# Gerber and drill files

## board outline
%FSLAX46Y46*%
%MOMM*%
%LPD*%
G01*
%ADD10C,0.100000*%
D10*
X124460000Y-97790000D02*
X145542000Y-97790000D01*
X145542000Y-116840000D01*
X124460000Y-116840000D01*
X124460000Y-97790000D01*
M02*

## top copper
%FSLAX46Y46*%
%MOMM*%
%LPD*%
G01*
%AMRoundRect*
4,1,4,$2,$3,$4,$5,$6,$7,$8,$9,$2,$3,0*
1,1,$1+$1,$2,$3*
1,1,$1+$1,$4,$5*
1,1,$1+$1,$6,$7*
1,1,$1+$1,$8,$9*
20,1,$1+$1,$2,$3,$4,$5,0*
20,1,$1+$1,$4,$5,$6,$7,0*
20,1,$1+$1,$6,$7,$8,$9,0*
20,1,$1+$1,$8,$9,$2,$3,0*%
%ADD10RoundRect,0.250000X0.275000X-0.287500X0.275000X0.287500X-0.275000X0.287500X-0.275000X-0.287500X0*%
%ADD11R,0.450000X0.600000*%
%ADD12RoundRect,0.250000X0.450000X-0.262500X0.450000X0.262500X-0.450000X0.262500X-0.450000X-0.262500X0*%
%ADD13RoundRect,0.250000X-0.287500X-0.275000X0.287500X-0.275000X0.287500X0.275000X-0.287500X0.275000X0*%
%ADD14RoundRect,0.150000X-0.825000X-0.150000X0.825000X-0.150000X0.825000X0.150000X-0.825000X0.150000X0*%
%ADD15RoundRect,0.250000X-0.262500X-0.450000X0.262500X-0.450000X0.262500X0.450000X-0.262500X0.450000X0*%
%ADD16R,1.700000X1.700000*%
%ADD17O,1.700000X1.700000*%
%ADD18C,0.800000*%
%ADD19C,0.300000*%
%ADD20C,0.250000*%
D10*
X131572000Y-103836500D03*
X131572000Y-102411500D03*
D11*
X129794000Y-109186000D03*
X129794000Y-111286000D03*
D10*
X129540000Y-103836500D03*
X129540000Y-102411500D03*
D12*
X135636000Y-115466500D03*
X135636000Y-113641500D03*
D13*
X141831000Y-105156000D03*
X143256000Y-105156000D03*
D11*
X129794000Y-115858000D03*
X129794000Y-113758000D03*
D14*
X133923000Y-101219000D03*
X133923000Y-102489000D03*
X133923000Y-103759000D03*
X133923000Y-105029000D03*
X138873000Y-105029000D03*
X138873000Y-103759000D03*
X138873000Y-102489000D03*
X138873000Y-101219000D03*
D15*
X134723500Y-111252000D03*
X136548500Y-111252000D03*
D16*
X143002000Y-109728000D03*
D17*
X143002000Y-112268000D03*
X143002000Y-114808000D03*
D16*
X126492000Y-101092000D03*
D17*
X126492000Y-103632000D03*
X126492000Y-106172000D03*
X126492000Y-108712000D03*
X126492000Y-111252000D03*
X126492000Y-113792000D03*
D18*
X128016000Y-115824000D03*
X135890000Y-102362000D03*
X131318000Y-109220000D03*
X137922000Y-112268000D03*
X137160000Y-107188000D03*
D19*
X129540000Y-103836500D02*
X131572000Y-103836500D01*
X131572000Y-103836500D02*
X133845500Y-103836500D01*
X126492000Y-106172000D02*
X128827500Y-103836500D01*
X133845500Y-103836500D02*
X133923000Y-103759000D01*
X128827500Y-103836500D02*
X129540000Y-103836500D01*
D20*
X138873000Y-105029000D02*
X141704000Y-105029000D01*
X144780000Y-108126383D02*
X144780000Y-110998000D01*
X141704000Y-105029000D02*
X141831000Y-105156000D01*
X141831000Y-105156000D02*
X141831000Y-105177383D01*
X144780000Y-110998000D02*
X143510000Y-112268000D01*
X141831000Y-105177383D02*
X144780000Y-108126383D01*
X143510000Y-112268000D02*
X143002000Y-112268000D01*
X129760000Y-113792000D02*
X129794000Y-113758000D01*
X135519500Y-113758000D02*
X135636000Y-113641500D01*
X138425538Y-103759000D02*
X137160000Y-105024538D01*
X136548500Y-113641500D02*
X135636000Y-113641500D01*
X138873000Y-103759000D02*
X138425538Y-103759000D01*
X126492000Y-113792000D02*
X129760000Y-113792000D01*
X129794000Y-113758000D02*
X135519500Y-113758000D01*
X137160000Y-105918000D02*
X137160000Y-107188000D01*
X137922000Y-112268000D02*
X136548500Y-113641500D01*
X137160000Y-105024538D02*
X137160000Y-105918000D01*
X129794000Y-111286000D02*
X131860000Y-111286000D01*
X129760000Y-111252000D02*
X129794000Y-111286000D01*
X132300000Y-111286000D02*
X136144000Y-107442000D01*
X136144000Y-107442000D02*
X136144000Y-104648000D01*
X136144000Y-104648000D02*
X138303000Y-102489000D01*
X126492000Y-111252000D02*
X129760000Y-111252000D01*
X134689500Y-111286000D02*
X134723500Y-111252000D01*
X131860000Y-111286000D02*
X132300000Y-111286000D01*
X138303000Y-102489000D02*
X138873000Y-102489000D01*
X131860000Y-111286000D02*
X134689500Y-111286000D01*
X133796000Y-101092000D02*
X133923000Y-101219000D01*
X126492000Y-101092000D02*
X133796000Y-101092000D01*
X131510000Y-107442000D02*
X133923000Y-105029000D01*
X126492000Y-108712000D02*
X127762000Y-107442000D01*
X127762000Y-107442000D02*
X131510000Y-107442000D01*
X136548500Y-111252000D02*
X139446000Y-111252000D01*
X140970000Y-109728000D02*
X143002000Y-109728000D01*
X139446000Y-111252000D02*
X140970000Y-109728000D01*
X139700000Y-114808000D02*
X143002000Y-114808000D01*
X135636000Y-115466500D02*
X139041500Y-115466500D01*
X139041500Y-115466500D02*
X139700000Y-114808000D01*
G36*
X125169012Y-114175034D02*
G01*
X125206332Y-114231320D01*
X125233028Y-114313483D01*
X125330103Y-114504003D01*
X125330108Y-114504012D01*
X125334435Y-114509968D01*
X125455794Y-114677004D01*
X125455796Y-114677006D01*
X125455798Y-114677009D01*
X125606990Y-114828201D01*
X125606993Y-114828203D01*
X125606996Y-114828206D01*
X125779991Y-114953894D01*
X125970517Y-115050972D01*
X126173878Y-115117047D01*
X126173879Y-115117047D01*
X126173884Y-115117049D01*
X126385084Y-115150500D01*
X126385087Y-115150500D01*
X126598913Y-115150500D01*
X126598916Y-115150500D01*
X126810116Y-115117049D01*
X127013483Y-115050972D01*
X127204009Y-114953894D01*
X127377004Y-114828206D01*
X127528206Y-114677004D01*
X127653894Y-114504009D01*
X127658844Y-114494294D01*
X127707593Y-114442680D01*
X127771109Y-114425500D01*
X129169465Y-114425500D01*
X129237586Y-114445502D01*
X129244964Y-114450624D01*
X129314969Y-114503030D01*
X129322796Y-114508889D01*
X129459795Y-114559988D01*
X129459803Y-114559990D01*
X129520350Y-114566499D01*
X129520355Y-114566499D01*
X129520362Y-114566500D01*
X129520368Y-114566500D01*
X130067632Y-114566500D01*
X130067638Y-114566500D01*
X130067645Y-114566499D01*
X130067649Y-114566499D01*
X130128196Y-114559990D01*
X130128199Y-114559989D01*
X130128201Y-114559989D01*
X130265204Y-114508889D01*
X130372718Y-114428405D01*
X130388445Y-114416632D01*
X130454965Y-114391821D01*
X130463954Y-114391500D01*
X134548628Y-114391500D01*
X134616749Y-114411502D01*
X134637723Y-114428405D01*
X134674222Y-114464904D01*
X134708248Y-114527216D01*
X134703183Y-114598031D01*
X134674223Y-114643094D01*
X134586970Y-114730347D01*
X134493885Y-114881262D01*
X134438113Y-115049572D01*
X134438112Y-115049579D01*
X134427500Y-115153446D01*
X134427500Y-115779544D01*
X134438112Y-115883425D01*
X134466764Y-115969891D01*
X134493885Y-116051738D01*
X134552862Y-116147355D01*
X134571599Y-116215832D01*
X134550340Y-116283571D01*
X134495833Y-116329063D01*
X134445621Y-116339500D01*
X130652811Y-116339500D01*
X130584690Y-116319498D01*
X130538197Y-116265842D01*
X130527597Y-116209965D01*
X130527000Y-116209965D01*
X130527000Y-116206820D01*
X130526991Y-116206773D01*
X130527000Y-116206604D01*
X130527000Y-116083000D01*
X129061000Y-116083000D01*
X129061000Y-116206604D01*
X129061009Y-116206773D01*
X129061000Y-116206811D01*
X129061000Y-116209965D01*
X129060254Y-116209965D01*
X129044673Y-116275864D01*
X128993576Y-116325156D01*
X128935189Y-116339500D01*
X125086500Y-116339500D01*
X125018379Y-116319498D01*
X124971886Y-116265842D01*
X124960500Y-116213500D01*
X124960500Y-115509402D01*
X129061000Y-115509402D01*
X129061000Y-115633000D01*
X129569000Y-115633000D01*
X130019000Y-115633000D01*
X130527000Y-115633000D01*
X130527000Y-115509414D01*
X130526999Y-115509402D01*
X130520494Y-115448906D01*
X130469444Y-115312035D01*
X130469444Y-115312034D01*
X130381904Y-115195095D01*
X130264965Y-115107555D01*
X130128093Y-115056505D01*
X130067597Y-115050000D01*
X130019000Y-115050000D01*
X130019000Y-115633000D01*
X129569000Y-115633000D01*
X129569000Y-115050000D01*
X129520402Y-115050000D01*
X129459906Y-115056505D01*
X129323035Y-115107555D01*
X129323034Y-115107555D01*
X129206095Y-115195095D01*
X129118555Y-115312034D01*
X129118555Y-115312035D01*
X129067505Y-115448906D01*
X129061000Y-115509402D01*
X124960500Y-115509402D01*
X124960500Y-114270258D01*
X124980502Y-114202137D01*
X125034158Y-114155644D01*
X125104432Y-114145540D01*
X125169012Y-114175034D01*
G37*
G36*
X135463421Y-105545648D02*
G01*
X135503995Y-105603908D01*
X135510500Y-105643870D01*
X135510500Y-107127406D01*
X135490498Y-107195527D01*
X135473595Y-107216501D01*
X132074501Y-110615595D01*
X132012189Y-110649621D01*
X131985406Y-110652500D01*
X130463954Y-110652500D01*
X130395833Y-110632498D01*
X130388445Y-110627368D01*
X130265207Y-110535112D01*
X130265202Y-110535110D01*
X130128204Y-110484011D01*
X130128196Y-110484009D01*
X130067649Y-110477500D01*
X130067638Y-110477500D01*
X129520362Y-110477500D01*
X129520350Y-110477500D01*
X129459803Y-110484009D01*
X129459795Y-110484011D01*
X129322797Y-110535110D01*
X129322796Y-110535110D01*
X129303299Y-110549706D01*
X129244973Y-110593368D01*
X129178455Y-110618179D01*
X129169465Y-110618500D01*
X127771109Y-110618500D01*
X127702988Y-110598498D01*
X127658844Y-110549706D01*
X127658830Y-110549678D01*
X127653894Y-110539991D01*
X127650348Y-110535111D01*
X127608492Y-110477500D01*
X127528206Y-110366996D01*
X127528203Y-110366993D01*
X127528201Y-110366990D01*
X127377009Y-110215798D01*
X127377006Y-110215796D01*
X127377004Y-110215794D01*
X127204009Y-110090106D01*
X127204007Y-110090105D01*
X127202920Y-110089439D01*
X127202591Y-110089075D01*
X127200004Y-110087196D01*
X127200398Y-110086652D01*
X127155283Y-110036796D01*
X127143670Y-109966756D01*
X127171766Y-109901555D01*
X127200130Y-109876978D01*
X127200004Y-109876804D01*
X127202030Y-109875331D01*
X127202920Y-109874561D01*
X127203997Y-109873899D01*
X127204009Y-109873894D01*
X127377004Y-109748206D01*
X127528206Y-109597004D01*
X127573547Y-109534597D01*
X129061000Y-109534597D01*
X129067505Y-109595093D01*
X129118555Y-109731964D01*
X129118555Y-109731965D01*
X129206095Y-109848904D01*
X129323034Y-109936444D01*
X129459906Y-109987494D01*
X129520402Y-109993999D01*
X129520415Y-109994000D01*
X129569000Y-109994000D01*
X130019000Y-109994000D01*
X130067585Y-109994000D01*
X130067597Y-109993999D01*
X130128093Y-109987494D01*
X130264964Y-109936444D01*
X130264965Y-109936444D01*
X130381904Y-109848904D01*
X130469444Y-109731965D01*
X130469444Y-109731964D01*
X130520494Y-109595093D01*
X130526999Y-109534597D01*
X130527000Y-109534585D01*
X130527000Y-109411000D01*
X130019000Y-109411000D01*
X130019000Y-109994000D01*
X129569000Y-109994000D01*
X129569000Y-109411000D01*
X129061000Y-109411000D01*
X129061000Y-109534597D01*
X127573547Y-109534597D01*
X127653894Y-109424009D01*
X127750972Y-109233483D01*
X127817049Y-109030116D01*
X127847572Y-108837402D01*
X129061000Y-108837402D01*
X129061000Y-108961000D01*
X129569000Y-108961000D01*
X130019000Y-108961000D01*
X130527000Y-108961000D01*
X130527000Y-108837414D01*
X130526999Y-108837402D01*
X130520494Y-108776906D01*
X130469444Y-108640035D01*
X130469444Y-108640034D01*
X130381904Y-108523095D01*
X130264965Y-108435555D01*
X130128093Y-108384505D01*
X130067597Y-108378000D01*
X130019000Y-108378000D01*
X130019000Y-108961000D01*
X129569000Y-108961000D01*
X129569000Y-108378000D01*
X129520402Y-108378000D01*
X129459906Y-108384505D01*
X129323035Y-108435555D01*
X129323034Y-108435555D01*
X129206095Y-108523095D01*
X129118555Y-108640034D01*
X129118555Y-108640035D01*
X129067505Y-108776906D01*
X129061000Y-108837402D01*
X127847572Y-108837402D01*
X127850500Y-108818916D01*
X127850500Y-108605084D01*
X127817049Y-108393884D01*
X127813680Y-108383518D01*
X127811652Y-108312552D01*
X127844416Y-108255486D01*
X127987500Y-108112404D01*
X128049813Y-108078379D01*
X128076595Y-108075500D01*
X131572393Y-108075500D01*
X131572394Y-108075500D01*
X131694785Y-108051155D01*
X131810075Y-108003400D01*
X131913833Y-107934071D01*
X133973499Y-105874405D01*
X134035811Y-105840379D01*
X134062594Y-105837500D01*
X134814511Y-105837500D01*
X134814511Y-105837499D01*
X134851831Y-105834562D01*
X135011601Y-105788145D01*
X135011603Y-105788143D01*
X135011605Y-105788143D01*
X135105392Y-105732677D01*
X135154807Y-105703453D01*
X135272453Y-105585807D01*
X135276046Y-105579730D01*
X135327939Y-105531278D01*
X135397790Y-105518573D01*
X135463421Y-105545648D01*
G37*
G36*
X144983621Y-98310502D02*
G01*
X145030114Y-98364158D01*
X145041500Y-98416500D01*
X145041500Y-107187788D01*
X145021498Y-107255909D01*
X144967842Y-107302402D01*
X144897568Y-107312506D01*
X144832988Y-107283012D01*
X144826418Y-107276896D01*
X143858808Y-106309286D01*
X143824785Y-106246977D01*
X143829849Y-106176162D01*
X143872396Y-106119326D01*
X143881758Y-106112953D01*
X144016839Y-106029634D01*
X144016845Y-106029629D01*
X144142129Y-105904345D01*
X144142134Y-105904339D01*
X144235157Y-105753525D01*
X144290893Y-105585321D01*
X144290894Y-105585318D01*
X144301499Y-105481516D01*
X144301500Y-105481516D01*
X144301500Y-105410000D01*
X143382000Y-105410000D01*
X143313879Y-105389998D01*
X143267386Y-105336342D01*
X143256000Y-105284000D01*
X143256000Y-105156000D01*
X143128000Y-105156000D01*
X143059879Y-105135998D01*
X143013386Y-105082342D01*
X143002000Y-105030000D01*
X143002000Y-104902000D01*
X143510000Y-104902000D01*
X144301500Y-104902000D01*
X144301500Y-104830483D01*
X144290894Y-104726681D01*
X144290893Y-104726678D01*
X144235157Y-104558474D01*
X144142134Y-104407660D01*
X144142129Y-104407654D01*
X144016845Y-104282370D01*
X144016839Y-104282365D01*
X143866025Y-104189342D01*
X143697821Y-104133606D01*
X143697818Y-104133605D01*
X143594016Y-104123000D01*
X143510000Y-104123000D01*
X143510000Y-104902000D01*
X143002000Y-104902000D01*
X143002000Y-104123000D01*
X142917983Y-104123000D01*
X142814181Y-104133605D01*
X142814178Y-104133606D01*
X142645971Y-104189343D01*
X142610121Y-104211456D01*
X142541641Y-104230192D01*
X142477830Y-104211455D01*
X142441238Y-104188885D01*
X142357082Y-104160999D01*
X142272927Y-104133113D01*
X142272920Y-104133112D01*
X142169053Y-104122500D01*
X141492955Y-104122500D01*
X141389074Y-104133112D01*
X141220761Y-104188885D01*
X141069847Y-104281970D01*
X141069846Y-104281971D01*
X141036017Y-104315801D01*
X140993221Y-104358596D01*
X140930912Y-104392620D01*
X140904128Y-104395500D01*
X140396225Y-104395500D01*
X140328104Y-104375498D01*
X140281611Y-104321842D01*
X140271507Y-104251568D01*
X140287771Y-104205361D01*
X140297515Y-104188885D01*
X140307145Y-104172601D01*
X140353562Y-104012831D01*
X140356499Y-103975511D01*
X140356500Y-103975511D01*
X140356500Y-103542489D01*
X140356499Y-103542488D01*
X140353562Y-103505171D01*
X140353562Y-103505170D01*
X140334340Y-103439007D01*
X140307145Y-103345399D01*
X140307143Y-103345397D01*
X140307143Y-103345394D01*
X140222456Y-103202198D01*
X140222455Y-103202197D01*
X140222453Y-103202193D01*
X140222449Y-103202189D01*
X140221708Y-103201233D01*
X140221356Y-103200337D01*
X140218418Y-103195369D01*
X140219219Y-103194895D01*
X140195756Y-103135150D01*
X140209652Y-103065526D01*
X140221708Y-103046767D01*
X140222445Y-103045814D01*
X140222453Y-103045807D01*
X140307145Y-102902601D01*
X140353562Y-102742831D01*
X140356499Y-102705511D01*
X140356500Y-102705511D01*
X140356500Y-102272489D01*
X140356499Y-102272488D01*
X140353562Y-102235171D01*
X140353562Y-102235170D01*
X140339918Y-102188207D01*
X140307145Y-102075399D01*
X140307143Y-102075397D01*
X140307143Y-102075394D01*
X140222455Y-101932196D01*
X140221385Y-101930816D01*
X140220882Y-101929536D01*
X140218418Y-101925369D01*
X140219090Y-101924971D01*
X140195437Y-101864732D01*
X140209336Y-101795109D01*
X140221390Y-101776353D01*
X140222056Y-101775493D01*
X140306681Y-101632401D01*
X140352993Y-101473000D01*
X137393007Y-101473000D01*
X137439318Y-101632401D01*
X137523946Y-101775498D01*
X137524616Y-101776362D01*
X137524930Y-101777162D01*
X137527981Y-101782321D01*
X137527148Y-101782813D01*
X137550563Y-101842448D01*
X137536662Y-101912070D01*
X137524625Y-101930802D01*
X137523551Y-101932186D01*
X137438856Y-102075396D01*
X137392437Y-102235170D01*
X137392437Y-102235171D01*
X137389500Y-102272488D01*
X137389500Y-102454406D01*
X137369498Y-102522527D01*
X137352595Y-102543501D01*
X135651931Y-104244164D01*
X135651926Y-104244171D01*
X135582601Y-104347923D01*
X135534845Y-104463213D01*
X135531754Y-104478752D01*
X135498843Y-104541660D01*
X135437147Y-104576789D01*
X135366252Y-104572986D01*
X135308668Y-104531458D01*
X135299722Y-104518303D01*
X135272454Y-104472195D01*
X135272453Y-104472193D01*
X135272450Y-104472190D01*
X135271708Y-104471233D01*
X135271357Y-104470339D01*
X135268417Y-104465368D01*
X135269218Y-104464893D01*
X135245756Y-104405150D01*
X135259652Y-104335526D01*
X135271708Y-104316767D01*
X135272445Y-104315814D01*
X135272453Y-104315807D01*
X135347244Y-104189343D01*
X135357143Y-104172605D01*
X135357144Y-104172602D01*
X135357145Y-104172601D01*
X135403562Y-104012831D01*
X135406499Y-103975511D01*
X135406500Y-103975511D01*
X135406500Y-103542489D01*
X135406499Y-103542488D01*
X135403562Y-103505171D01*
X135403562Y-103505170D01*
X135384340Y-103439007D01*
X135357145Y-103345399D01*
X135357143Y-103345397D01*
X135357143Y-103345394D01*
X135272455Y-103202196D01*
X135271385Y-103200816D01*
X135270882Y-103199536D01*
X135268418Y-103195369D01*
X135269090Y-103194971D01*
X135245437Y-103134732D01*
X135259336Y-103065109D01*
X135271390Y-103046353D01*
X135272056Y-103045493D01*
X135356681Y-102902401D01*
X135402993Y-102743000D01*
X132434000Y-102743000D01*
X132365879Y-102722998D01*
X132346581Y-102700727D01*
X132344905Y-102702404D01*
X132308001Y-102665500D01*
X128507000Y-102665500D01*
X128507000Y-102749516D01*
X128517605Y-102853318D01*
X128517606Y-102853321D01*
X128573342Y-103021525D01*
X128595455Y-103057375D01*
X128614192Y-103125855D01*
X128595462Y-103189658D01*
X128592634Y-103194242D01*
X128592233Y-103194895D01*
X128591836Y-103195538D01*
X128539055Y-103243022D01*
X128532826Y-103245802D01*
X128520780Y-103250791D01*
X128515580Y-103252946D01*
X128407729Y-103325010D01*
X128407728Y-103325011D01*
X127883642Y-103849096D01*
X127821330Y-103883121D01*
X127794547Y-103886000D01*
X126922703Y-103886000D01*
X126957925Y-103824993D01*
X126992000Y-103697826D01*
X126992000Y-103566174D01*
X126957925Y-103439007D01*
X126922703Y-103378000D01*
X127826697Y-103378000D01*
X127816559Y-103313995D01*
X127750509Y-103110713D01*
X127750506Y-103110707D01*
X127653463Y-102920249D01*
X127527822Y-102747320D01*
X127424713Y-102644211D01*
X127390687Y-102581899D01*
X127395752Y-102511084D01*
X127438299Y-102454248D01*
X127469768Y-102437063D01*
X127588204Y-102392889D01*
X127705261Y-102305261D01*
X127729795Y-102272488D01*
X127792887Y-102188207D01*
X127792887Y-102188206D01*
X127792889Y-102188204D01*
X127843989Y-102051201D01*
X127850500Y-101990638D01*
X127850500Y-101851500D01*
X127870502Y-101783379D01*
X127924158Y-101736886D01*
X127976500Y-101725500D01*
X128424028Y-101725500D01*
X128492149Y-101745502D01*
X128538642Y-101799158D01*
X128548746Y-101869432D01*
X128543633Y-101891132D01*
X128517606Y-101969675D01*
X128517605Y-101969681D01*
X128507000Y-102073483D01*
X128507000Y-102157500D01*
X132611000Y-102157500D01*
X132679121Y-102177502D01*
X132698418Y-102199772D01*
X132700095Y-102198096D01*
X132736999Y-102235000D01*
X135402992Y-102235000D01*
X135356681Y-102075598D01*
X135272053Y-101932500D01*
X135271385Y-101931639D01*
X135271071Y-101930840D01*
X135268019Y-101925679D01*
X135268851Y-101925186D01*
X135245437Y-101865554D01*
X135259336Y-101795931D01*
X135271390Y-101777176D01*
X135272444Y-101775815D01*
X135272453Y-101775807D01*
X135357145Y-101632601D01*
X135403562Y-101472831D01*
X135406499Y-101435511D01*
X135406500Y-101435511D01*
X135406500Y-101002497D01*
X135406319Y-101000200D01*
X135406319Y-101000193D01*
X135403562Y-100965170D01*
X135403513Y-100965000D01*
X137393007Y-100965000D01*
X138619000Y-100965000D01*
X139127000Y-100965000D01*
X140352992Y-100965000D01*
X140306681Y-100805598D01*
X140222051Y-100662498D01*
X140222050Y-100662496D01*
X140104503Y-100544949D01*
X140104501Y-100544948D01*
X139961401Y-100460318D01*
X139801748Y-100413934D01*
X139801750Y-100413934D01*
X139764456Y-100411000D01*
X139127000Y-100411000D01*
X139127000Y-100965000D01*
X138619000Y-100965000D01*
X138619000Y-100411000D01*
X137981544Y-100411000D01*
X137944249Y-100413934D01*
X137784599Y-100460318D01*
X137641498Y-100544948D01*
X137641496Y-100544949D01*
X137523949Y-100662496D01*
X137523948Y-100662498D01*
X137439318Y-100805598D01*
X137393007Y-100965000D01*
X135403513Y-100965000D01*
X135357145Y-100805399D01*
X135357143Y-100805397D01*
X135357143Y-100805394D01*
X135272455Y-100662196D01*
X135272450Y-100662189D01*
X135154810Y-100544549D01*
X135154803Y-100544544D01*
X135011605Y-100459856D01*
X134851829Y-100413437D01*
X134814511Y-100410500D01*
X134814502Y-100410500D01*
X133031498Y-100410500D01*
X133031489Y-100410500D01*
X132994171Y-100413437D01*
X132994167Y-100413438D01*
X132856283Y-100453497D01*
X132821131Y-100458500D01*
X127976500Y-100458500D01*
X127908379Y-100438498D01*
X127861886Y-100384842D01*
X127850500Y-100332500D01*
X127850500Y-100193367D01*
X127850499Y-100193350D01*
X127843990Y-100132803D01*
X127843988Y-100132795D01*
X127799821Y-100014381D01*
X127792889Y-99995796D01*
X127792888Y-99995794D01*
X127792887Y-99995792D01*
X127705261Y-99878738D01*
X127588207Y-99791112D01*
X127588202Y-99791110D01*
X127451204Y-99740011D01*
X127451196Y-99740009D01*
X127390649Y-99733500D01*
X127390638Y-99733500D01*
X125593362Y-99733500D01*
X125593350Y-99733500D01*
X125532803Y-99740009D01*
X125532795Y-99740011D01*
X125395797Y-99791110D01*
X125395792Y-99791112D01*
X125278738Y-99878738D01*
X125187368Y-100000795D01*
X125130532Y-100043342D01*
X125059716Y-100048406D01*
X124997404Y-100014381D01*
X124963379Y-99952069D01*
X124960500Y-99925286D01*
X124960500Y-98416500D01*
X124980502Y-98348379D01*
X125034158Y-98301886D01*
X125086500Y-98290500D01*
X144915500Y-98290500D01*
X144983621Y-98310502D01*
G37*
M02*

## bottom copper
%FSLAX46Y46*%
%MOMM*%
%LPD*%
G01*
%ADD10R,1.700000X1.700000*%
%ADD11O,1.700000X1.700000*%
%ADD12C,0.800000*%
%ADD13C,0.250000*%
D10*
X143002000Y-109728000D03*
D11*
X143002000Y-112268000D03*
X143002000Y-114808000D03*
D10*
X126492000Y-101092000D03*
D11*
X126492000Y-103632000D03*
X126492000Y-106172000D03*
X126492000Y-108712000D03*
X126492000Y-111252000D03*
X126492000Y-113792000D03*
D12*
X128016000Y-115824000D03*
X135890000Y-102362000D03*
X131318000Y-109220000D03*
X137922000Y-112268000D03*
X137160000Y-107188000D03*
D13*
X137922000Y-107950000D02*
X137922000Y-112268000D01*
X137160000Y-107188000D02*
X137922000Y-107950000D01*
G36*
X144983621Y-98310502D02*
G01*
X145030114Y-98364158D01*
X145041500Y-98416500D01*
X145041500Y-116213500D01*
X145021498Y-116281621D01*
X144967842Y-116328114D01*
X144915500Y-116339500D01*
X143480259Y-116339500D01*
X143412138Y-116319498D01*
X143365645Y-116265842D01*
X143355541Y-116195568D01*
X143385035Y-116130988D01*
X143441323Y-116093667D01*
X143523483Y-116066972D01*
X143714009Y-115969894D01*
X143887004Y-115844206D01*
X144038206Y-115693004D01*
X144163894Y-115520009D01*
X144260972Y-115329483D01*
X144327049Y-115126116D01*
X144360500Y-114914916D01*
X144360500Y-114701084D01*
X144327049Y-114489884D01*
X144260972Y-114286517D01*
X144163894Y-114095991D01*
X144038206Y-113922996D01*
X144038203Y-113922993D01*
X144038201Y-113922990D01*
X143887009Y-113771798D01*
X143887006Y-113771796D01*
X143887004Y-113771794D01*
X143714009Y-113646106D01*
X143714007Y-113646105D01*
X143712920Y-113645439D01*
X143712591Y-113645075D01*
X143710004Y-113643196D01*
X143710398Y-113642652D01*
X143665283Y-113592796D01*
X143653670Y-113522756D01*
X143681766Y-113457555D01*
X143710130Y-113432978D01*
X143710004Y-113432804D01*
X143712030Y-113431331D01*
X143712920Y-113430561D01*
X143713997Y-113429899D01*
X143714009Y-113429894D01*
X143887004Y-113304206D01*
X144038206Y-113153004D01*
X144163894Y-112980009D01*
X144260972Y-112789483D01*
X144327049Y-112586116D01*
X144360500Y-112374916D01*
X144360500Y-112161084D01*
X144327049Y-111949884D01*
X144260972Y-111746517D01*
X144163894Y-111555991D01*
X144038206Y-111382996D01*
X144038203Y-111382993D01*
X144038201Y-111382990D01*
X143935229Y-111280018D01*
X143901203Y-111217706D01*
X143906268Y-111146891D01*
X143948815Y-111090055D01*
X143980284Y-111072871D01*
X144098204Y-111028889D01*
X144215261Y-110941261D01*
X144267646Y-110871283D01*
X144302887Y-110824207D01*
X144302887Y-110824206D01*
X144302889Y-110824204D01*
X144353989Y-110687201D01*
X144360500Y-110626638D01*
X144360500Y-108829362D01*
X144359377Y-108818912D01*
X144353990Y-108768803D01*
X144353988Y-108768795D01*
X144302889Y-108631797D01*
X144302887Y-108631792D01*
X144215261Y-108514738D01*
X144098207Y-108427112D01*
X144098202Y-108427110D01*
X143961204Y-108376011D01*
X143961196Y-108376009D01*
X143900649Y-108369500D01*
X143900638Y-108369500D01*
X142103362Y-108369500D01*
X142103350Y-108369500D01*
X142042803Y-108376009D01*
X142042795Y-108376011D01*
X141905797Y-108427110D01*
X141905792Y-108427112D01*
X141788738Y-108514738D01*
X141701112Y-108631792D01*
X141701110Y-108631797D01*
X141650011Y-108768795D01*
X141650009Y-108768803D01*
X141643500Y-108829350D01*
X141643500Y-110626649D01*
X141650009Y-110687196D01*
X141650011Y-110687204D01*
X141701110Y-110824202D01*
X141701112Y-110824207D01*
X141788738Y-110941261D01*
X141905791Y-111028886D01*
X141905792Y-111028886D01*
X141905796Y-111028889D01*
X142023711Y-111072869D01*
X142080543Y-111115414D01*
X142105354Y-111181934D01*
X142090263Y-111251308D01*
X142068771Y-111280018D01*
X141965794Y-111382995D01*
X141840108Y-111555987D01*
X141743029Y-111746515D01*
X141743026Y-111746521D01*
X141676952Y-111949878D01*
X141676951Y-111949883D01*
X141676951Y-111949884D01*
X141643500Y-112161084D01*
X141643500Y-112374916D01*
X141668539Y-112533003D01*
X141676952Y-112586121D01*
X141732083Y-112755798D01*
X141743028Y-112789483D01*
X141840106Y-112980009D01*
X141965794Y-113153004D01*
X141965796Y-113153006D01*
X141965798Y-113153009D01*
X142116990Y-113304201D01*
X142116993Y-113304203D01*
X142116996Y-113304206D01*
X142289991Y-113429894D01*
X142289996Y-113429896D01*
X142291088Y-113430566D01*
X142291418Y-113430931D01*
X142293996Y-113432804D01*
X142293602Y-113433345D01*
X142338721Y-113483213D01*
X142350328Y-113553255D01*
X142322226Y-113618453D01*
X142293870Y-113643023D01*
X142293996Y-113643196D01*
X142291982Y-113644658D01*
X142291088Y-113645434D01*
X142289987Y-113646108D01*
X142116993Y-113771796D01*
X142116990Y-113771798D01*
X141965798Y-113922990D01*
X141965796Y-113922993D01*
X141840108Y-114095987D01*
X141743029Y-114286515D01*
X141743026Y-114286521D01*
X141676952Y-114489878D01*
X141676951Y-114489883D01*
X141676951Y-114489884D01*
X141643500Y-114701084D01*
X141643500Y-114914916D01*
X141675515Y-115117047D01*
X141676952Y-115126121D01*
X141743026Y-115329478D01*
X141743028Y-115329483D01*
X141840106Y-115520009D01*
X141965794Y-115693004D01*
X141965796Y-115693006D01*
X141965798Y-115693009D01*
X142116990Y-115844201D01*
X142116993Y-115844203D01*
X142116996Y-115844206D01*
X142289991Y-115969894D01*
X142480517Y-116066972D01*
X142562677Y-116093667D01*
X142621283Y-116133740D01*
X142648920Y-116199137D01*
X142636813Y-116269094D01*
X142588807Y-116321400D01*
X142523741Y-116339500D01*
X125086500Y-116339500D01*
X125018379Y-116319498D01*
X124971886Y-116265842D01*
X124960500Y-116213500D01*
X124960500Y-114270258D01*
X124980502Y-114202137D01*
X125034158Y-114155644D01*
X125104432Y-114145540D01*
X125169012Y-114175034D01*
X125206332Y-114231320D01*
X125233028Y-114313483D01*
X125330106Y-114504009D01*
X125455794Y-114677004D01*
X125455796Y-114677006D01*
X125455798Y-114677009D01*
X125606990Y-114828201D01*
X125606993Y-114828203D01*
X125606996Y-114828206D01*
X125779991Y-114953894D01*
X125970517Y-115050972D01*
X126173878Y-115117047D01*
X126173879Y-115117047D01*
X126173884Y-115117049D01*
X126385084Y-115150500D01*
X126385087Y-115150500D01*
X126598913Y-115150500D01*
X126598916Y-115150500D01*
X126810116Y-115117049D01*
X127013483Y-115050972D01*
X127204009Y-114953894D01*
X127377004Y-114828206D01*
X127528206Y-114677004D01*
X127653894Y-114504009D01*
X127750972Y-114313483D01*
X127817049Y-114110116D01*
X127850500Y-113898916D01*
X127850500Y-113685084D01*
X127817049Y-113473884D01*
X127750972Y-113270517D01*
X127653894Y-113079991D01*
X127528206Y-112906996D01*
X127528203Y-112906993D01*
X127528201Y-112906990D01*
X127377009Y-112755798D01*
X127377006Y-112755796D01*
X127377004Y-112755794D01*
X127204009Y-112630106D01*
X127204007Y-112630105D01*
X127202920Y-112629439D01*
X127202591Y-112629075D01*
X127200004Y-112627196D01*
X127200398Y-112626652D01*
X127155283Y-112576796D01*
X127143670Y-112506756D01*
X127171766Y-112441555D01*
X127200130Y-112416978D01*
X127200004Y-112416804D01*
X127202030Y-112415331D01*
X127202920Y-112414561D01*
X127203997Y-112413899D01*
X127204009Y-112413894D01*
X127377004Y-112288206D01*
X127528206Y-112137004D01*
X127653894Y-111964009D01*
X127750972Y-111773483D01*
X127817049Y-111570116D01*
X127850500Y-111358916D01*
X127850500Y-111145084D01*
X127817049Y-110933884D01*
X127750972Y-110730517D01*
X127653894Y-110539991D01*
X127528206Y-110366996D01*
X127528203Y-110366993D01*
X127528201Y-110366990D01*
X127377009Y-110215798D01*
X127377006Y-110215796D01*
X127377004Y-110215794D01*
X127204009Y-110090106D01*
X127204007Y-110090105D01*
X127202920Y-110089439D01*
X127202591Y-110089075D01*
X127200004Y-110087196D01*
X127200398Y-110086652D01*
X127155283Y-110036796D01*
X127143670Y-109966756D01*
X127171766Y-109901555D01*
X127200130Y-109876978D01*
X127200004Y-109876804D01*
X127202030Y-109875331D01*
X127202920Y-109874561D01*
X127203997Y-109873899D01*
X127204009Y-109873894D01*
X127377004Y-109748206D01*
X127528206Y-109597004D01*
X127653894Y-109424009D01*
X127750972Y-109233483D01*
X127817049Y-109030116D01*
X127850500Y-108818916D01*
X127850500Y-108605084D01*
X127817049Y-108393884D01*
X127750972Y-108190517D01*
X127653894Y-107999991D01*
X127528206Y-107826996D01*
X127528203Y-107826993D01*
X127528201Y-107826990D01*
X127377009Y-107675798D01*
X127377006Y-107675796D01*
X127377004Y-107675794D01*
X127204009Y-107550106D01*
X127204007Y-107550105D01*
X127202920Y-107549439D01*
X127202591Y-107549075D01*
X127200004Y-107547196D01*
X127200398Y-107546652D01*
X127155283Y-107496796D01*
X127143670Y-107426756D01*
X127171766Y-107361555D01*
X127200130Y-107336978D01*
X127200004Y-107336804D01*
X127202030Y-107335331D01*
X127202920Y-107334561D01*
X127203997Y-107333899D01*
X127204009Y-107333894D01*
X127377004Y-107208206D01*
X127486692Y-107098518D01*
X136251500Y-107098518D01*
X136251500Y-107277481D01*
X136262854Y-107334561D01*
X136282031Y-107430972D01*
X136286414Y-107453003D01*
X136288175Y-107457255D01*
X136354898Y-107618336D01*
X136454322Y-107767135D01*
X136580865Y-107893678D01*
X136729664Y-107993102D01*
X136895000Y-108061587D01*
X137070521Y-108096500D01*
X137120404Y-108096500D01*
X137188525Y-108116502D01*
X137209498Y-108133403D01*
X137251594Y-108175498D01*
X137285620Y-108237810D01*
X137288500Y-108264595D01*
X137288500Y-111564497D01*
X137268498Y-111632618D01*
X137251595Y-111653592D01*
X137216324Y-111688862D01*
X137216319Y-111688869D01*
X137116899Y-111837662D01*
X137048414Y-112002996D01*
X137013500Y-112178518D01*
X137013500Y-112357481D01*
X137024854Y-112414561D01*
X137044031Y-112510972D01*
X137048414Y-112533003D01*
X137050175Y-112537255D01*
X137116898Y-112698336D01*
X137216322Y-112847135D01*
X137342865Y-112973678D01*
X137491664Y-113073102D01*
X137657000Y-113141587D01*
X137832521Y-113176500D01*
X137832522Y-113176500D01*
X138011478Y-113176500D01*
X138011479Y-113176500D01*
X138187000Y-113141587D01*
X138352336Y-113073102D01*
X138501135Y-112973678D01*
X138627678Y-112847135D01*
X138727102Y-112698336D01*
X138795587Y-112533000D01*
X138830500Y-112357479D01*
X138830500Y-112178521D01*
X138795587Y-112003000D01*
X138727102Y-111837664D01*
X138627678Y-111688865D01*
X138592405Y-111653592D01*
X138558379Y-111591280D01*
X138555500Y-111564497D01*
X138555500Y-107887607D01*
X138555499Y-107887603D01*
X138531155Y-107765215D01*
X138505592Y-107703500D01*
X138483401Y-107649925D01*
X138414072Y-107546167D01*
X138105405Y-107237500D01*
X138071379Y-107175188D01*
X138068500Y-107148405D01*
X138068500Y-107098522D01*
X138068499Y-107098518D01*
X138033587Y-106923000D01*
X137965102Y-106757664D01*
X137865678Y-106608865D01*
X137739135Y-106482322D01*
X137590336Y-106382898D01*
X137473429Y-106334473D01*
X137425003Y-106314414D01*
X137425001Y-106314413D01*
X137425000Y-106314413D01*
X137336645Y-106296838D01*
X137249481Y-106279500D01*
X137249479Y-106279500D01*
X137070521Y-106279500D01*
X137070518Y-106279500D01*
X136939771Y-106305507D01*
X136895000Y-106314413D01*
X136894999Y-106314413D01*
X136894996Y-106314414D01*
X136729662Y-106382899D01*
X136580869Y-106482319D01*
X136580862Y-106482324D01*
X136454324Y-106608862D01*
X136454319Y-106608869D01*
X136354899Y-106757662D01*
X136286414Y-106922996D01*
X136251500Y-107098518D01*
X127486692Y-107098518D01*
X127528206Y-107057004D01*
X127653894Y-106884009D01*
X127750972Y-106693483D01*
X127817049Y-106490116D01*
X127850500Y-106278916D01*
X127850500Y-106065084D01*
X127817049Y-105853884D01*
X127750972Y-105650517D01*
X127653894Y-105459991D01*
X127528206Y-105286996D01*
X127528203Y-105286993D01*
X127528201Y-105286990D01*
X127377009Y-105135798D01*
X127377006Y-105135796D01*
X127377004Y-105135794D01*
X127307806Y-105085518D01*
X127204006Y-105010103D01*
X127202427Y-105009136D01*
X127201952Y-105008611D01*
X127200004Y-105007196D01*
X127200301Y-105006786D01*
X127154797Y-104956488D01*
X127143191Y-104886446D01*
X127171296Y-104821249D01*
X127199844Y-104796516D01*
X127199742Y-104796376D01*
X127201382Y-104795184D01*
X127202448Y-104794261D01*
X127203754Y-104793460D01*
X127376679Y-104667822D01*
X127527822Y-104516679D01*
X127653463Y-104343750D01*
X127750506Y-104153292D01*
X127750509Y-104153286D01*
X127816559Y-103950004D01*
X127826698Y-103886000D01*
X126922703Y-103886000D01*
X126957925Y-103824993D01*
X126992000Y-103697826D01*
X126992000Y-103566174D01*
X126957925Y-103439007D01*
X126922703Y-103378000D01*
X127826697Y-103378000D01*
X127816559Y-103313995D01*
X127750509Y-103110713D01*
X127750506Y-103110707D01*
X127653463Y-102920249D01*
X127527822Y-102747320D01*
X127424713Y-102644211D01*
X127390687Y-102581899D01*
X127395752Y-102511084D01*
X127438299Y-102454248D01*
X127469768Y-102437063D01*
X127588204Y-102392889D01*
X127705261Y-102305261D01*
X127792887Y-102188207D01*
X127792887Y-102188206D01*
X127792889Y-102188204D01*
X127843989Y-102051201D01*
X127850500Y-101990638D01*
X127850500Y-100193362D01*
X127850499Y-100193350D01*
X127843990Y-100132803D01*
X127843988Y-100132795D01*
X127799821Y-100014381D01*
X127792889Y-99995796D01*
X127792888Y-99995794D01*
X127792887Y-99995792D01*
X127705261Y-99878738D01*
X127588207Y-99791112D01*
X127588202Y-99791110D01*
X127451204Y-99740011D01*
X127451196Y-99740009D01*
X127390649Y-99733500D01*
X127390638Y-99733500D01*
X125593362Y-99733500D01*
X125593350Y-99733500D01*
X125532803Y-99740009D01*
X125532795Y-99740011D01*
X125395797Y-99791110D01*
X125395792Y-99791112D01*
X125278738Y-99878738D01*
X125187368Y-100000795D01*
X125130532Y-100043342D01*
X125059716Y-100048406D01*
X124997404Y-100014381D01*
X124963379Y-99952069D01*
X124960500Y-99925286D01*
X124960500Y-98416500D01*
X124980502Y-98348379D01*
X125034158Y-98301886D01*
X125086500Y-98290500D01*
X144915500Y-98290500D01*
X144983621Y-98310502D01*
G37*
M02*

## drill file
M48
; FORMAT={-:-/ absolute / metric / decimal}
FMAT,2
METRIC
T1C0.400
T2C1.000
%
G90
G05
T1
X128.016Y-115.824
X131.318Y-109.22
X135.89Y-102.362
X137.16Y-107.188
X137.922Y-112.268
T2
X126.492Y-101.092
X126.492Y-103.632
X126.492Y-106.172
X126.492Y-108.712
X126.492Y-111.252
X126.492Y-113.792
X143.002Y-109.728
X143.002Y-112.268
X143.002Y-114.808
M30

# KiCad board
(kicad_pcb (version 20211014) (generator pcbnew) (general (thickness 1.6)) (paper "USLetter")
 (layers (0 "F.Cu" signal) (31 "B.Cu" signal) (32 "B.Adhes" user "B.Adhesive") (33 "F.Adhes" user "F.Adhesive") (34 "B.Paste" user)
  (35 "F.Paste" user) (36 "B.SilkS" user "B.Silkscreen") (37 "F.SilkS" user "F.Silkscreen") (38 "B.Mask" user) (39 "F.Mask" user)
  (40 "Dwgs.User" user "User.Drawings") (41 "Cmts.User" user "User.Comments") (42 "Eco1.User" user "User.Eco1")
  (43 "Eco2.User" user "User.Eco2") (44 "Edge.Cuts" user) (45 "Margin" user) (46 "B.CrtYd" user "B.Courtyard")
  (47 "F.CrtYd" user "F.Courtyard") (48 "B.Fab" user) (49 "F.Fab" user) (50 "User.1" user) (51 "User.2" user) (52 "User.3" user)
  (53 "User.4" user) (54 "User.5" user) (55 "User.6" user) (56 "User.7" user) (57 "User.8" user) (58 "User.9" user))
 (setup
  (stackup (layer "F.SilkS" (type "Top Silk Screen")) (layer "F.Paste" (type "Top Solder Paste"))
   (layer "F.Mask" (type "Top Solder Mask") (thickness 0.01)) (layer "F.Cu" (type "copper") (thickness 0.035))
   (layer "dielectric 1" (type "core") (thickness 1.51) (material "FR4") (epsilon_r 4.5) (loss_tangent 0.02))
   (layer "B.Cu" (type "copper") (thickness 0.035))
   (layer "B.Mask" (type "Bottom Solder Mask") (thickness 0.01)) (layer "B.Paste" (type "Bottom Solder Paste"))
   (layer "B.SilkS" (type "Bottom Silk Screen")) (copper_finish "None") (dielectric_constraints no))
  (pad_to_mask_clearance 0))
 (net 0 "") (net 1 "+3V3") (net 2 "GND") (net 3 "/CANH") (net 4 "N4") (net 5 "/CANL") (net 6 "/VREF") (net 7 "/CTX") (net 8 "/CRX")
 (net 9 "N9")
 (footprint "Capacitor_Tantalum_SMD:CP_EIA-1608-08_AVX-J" (layer "F.Cu") (at 131.572 103.124 90)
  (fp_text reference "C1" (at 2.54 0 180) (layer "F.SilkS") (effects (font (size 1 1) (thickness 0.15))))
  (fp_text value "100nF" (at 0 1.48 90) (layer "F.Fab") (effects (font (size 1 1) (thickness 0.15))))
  (pad "1" smd roundrect (at -0.7125 0 90) (size 1.075 1.05) (layers "F.Cu" "F.Paste" "F.Mask") (roundrect_rratio 0.238095) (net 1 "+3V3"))
  (pad "2" smd roundrect (at 0.7125 0 90) (size 1.075 1.05) (layers "F.Cu" "F.Paste" "F.Mask") (roundrect_rratio 0.238095) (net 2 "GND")))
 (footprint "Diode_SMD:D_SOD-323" (layer "F.Cu") (at 129.794 110.236 -90)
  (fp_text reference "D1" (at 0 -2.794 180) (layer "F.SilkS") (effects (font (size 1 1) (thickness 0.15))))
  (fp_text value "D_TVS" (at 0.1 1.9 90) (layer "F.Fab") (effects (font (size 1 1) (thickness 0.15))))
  (pad "1" smd rect (at -1.05 0 270) (size 0.6 0.45) (layers "F.Cu" "F.Paste" "F.Mask") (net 2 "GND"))
  (pad "2" smd rect (at 1.05 0 270) (size 0.6 0.45) (layers "F.Cu" "F.Paste" "F.Mask") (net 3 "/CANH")))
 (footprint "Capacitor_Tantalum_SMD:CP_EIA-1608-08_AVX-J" (layer "F.Cu") (at 129.54 103.124 90)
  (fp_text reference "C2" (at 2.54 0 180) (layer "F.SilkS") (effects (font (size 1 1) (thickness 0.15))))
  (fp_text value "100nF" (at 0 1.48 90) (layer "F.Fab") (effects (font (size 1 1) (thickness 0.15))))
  (pad "1" smd roundrect (at -0.7125 0 90) (size 1.075 1.05) (layers "F.Cu" "F.Paste" "F.Mask") (roundrect_rratio 0.238095) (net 1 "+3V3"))
  (pad "2" smd roundrect (at 0.7125 0 90) (size 1.075 1.05) (layers "F.Cu" "F.Paste" "F.Mask") (roundrect_rratio 0.238095) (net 2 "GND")))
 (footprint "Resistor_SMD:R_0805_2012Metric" (layer "F.Cu") (at 135.636 114.554 90)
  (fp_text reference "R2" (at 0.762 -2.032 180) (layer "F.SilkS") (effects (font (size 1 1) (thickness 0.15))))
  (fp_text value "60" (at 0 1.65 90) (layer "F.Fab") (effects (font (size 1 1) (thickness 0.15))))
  (pad "1" smd roundrect (at -0.9125 0 90) (size 1.025 1.4) (layers "F.Cu" "F.Paste" "F.Mask") (roundrect_rratio 0.243902) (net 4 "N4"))
  (pad "2" smd roundrect (at 0.9125 0 90) (size 1.025 1.4) (layers "F.Cu" "F.Paste" "F.Mask") (roundrect_rratio 0.243902) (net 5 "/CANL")))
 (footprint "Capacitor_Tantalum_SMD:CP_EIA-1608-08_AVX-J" (layer "F.Cu") (at 142.5435 105.156)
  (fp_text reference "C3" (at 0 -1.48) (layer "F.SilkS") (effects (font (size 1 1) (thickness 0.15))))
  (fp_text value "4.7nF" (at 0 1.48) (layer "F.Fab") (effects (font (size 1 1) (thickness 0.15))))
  (pad "1" smd roundrect (at -0.7125 0) (size 1.075 1.05) (layers "F.Cu" "F.Paste" "F.Mask") (roundrect_rratio 0.238095) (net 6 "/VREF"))
  (pad "2" smd roundrect (at 0.7125 0) (size 1.075 1.05) (layers "F.Cu" "F.Paste" "F.Mask") (roundrect_rratio 0.238095) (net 2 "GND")))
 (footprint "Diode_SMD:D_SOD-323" (layer "F.Cu") (at 129.794 114.808 90)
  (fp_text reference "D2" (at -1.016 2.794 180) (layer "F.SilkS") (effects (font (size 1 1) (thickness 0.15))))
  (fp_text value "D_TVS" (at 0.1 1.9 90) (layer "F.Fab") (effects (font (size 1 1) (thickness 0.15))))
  (pad "1" smd rect (at -1.05 0 90) (size 0.6 0.45) (layers "F.Cu" "F.Paste" "F.Mask") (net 2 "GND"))
  (pad "2" smd rect (at 1.05 0 90) (size 0.6 0.45) (layers "F.Cu" "F.Paste" "F.Mask") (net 5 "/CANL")))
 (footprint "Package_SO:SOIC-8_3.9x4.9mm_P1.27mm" (layer "F.Cu") (at 136.398 103.124)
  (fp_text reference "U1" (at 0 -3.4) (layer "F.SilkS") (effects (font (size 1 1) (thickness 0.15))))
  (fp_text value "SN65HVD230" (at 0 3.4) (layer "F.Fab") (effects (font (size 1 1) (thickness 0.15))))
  (pad "1" smd roundrect (at -2.475 -1.905) (size 1.95 0.6) (layers "F.Cu" "F.Paste" "F.Mask") (roundrect_rratio 0.25) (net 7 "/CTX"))
  (pad "2" smd roundrect (at -2.475 -0.635) (size 1.95 0.6) (layers "F.Cu" "F.Paste" "F.Mask") (roundrect_rratio 0.25) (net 2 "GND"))
  (pad "3" smd roundrect (at -2.475 0.635) (size 1.95 0.6) (layers "F.Cu" "F.Paste" "F.Mask") (roundrect_rratio 0.25) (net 1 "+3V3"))
  (pad "4" smd roundrect (at -2.475 1.905) (size 1.95 0.6) (layers "F.Cu" "F.Paste" "F.Mask") (roundrect_rratio 0.25) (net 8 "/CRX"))
  (pad "5" smd roundrect (at 2.475 1.905) (size 1.95 0.6) (layers "F.Cu" "F.Paste" "F.Mask") (roundrect_rratio 0.25) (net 6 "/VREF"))
  (pad "6" smd roundrect (at 2.475 0.635) (size 1.95 0.6) (layers "F.Cu" "F.Paste" "F.Mask") (roundrect_rratio 0.25) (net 5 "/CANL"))
  (pad "7" smd roundrect (at 2.475 -0.635) (size 1.95 0.6) (layers "F.Cu" "F.Paste" "F.Mask") (roundrect_rratio 0.25) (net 3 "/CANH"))
  (pad "8" smd roundrect (at 2.475 -1.905) (size 1.95 0.6) (layers "F.Cu" "F.Paste" "F.Mask") (roundrect_rratio 0.25) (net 2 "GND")))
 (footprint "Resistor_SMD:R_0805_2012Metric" (layer "F.Cu") (at 135.636 111.252)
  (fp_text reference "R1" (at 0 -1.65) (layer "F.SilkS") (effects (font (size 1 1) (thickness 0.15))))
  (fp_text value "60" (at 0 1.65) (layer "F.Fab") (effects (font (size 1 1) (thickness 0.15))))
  (pad "1" smd roundrect (at -0.9125 0) (size 1.025 1.4) (layers "F.Cu" "F.Paste" "F.Mask") (roundrect_rratio 0.243902) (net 3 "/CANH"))
  (pad "2" smd roundrect (at 0.9125 0) (size 1.025 1.4) (layers "F.Cu" "F.Paste" "F.Mask") (roundrect_rratio 0.243902) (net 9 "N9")))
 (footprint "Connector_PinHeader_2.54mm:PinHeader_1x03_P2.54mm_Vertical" (layer "F.Cu") (at 143.002 109.728)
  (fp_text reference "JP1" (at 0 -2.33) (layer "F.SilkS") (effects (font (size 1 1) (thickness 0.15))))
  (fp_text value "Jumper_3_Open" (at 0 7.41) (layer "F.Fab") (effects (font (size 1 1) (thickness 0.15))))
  (pad "1" thru_hole rect (at 0 0) (size 1.7 1.7) (drill 1) (layers *.Cu *.Mask) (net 9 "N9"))
  (pad "2" thru_hole oval (at 0 2.54) (size 1.7 1.7) (drill 1) (layers *.Cu *.Mask) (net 6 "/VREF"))
  (pad "3" thru_hole oval (at 0 5.08) (size 1.7 1.7) (drill 1) (layers *.Cu *.Mask) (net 4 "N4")))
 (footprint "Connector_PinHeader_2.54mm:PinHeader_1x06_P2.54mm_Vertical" (layer "B.Cu") (at 126.492 101.092 180)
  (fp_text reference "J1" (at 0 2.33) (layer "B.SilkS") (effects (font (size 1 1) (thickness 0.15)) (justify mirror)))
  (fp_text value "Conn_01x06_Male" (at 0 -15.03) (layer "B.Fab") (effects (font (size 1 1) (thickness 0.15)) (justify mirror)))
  (pad "1" thru_hole rect (at 0 0 180) (size 1.7 1.7) (drill 1) (layers *.Cu *.Mask) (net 7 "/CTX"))
  (pad "2" thru_hole oval (at 0 -2.54 180) (size 1.7 1.7) (drill 1) (layers *.Cu *.Mask) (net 2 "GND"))
  (pad "3" thru_hole oval (at 0 -5.08 180) (size 1.7 1.7) (drill 1) (layers *.Cu *.Mask) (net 1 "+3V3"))
  (pad "4" thru_hole oval (at 0 -7.62 180) (size 1.7 1.7) (drill 1) (layers *.Cu *.Mask) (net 8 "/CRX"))
  (pad "5" thru_hole oval (at 0 -10.16 180) (size 1.7 1.7) (drill 1) (layers *.Cu *.Mask) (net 3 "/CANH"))
  (pad "6" thru_hole oval (at 0 -12.7 180) (size 1.7 1.7) (drill 1) (layers *.Cu *.Mask) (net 5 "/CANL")))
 (gr_rect (start 124.46 116.84) (end 145.542 97.79) (layer "Edge.Cuts") (width 0.1) (fill none))
 (segment (start 129.54 103.8365) (end 131.572 103.8365) (width 0.3) (layer "F.Cu") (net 1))
 (segment (start 131.572 103.8365) (end 133.8455 103.8365) (width 0.3) (layer "F.Cu") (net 1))
 (segment (start 126.492 106.172) (end 128.8275 103.8365) (width 0.3) (layer "F.Cu") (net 1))
 (segment (start 133.8455 103.8365) (end 133.923 103.759) (width 0.3) (layer "F.Cu") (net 1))
 (segment (start 128.8275 103.8365) (end 129.54 103.8365) (width 0.3) (layer "F.Cu") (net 1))
 (via (at 128.016 115.824) (size 0.8) (drill 0.4) (layers "F.Cu" "B.Cu") (free) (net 2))
 (via (at 135.89 102.362) (size 0.8) (drill 0.4) (layers "F.Cu" "B.Cu") (free) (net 2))
 (via (at 131.318 109.22) (size 0.8) (drill 0.4) (layers "F.Cu" "B.Cu") (free) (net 2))
 (segment (start 138.873 105.029) (end 141.704 105.029) (width 0.25) (layer "F.Cu") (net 6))
 (segment (start 144.78 108.126383) (end 144.78 110.998) (width 0.25) (layer "F.Cu") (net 6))
 (segment (start 141.704 105.029) (end 141.831 105.156) (width 0.25) (layer "F.Cu") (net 6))
 (segment (start 141.831 105.156) (end 141.831 105.177383) (width 0.25) (layer "F.Cu") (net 6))
 (segment (start 144.78 110.998) (end 143.51 112.268) (width 0.25) (layer "F.Cu") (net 6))
 (segment (start 141.831 105.177383) (end 144.78 108.126383) (width 0.25) (layer "F.Cu") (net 6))
 (segment (start 143.51 112.268) (end 143.002 112.268) (width 0.25) (layer "F.Cu") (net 6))
 (segment (start 129.76 113.792) (end 129.794 113.758) (width 0.25) (layer "F.Cu") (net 5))
 (segment (start 135.5195 113.758) (end 135.636 113.6415) (width 0.25) (layer "F.Cu") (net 5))
 (segment (start 138.425538 103.759) (end 137.16 105.024538) (width 0.25) (layer "F.Cu") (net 5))
 (segment (start 136.5485 113.6415) (end 135.636 113.6415) (width 0.25) (layer "F.Cu") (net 5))
 (segment (start 138.873 103.759) (end 138.425538 103.759) (width 0.25) (layer "F.Cu") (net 5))
 (segment (start 126.492 113.792) (end 129.76 113.792) (width 0.25) (layer "F.Cu") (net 5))
 (segment (start 129.794 113.758) (end 135.5195 113.758) (width 0.25) (layer "F.Cu") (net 5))
 (segment (start 137.16 105.918) (end 137.16 107.188) (width 0.25) (layer "F.Cu") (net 5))
 (segment (start 137.922 112.268) (end 136.5485 113.6415) (width 0.25) (layer "F.Cu") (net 5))
 (segment (start 137.16 105.024538) (end 137.16 105.918) (width 0.25) (layer "F.Cu") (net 5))
 (via (at 137.922 112.268) (size 0.8) (drill 0.4) (layers "F.Cu" "B.Cu") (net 5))
 (via (at 137.16 107.188) (size 0.8) (drill 0.4) (layers "F.Cu" "B.Cu") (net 5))
 (segment (start 137.922 107.95) (end 137.922 112.268) (width 0.25) (layer "B.Cu") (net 5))
 (segment (start 137.16 107.188) (end 137.922 107.95) (width 0.25) (layer "B.Cu") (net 5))
 (segment (start 129.794 111.286) (end 131.86 111.286) (width 0.25) (layer "F.Cu") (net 3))
 (segment (start 129.76 111.252) (end 129.794 111.286) (width 0.25) (layer "F.Cu") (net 3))
 (segment (start 132.3 111.286) (end 136.144 107.442) (width 0.25) (layer "F.Cu") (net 3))
 (segment (start 136.144 107.442) (end 136.144 104.648) (width 0.25) (layer "F.Cu") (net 3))
 (segment (start 136.144 104.648) (end 138.303 102.489) (width 0.25) (layer "F.Cu") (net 3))
 (segment (start 126.492 111.252) (end 129.76 111.252) (width 0.25) (layer "F.Cu") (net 3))
 (segment (start 134.6895 111.286) (end 134.7235 111.252) (width 0.25) (layer "F.Cu") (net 3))
 (segment (start 131.86 111.286) (end 132.3 111.286) (width 0.25) (layer "F.Cu") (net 3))
 (segment (start 138.303 102.489) (end 138.873 102.489) (width 0.25) (layer "F.Cu") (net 3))
 (segment (start 131.86 111.286) (end 134.6895 111.286) (width 0.25) (layer "F.Cu") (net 3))
 (segment (start 133.796 101.092) (end 133.923 101.219) (width 0.25) (layer "F.Cu") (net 7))
 (segment (start 126.492 101.092) (end 133.796 101.092) (width 0.25) (layer "F.Cu") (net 7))
 (segment (start 131.51 107.442) (end 133.923 105.029) (width 0.25) (layer "F.Cu") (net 8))
 (segment (start 126.492 108.712) (end 127.762 107.442) (width 0.25) (layer "F.Cu") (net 8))
 (segment (start 127.762 107.442) (end 131.51 107.442) (width 0.25) (layer "F.Cu") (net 8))
 (segment (start 136.5485 111.252) (end 139.446 111.252) (width 0.25) (layer "F.Cu") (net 9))
 (segment (start 140.97 109.728) (end 143.002 109.728) (width 0.25) (layer "F.Cu") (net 9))
 (segment (start 139.446 111.252) (end 140.97 109.728) (width 0.25) (layer "F.Cu") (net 9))
 (segment (start 139.7 114.808) (end 143.002 114.808) (width 0.25) (layer "F.Cu") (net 4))
 (segment (start 135.636 115.4665) (end 139.0415 115.4665) (width 0.25) (layer "F.Cu") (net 4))
 (segment (start 139.0415 115.4665) (end 139.7 114.808) (width 0.25) (layer "F.Cu") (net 4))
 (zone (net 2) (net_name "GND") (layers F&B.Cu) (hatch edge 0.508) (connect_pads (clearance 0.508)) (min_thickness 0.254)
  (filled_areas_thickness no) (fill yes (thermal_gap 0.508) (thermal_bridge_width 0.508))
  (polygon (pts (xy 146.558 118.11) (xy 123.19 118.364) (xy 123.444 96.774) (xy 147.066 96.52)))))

